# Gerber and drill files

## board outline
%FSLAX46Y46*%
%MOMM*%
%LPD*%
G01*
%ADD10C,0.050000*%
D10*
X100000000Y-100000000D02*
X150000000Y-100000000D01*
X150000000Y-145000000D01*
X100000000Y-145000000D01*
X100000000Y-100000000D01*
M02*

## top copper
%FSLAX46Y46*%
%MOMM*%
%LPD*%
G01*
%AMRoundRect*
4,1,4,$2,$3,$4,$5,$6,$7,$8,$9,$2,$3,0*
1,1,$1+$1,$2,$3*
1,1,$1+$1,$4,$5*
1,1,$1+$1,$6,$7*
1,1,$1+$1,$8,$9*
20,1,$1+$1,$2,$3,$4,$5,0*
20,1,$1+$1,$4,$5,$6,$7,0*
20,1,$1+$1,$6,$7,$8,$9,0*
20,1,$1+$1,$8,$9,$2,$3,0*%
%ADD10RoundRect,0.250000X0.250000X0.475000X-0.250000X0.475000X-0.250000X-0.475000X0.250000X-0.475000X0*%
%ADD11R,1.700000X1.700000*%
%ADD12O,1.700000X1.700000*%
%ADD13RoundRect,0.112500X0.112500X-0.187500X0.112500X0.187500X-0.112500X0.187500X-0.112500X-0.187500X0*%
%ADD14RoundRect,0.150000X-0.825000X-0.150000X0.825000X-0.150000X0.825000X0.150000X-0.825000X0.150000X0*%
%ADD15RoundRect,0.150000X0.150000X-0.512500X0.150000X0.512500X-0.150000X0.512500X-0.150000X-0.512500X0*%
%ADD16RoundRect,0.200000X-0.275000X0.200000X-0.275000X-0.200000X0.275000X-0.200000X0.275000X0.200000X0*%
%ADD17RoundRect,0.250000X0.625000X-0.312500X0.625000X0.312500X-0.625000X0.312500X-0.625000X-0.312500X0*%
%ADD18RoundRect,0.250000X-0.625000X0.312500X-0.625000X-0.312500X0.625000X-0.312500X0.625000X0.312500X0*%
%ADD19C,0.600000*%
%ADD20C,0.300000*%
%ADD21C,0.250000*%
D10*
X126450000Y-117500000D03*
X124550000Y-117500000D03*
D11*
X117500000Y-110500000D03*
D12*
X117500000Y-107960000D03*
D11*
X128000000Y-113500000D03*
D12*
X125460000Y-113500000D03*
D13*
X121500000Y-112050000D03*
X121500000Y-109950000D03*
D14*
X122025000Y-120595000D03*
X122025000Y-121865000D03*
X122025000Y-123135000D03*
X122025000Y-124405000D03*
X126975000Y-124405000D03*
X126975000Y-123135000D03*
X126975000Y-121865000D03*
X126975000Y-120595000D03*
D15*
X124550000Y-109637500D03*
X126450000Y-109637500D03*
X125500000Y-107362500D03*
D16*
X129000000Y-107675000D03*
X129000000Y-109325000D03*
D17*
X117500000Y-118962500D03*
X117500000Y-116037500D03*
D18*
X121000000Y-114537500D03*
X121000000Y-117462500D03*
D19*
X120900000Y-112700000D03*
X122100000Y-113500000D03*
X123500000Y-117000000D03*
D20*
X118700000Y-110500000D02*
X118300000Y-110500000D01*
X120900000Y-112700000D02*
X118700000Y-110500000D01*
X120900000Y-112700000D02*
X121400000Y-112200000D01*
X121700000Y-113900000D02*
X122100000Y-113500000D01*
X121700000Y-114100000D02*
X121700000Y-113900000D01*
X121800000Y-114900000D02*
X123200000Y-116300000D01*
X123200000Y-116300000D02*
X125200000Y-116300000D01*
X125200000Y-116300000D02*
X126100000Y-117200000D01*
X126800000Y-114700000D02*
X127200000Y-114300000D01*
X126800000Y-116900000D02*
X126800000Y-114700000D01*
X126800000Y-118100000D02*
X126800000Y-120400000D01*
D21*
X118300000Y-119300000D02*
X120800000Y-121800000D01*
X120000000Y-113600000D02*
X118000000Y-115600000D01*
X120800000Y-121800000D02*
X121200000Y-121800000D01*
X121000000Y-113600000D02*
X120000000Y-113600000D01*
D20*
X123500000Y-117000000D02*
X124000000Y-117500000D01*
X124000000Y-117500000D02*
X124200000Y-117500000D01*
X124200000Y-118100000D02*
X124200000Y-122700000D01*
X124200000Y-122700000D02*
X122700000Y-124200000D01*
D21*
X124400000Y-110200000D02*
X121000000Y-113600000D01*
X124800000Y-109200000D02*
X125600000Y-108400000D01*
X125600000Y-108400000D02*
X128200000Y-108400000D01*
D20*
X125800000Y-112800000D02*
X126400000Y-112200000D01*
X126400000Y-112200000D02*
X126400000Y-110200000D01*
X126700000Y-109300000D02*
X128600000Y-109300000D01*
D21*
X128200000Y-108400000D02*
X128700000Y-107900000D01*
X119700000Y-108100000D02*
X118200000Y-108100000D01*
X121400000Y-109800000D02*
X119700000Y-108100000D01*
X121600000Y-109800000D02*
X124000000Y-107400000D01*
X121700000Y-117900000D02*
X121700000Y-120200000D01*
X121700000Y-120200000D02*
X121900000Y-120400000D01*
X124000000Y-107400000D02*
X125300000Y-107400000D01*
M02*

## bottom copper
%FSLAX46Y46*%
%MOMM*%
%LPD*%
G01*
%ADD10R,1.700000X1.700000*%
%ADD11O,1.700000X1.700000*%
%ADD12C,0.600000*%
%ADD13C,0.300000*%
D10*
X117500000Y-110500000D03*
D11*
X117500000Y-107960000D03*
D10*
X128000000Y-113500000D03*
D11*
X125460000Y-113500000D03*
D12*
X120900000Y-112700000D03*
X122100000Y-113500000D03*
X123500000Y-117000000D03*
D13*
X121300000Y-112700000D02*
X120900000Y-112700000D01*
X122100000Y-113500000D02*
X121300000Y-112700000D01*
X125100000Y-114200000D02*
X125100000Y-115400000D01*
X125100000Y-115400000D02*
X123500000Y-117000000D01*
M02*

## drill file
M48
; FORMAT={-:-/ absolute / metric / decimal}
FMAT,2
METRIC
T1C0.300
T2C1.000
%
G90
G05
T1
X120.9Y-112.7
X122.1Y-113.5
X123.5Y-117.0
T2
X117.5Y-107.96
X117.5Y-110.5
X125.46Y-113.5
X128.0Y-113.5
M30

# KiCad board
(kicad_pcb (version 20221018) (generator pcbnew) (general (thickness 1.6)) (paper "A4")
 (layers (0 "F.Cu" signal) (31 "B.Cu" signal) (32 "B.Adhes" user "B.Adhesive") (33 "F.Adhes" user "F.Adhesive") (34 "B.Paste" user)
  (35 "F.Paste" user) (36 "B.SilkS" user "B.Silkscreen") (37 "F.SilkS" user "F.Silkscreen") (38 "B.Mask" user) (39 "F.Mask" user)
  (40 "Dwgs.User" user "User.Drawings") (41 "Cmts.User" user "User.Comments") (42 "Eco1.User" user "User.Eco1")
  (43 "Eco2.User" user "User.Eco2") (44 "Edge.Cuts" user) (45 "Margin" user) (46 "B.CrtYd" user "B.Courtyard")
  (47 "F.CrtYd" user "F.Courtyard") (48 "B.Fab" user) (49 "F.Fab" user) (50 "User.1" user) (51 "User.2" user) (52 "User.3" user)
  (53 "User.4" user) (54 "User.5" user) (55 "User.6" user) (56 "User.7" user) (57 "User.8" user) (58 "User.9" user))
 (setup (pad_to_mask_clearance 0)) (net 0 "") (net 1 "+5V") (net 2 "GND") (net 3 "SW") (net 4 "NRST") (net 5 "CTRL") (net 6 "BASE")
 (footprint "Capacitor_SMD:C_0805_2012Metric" (layer "F.Cu") (at 125.5 117.5 180)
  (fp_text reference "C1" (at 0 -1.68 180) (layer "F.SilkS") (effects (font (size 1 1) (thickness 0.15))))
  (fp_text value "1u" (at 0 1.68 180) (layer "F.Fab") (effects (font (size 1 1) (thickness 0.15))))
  (pad "1" smd roundrect (at -0.95 0 180) (size 1 1.45) (layers "F.Cu" "F.Paste" "F.Mask") (roundrect_rratio 0.25) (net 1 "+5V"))
  (pad "2" smd roundrect (at 0.95 0 180) (size 1 1.45) (layers "F.Cu" "F.Paste" "F.Mask") (roundrect_rratio 0.25) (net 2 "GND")))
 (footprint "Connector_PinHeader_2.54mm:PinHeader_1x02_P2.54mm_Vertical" (layer "F.Cu") (at 117.5 110.5 180)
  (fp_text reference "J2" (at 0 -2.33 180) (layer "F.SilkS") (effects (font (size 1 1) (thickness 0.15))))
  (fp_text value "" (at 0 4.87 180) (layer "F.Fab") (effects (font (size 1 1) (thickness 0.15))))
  (pad "1" thru_hole rect (at 0 0 180) (size 1.7 1.7) (drill 1) (layers "*.Cu" "*.Mask") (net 1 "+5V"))
  (pad "2" thru_hole oval (at 0 2.54 180) (size 1.7 1.7) (drill 1) (layers "*.Cu" "*.Mask") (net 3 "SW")))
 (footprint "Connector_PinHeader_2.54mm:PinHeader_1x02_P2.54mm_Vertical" (layer "F.Cu") (at 128 113.5 -90)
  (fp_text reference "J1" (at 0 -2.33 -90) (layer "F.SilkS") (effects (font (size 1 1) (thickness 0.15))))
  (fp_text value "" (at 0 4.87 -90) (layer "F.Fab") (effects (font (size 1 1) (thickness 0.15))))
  (pad "1" thru_hole rect (at 0 0 270) (size 1.7 1.7) (drill 1) (layers "*.Cu" "*.Mask") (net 1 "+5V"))
  (pad "2" thru_hole oval (at 0 2.54 270) (size 1.7 1.7) (drill 1) (layers "*.Cu" "*.Mask") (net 2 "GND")))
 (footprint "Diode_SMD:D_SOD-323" (layer "F.Cu") (at 121.5 111 90)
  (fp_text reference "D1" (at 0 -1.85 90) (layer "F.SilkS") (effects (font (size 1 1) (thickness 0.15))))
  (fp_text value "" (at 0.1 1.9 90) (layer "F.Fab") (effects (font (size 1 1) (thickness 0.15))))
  (pad "1" smd roundrect (at -1.05 0 90) (size 0.6 0.45) (layers "F.Cu" "F.Paste" "F.Mask") (roundrect_rratio 0.25) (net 1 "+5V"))
  (pad "2" smd roundrect (at 1.05 0 90) (size 0.6 0.45) (layers "F.Cu" "F.Paste" "F.Mask") (roundrect_rratio 0.25) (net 3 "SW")))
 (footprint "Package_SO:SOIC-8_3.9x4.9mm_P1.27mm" (layer "F.Cu") (at 124.5 122.5)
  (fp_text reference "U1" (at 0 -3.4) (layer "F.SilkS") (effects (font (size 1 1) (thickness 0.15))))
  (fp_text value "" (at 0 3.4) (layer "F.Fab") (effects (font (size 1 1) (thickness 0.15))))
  (pad "1" smd roundrect (at -2.475 -1.905) (size 1.95 0.6) (layers "F.Cu" "F.Paste" "F.Mask") (roundrect_rratio 0.25) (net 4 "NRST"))
  (pad "2" smd roundrect (at -2.475 -0.635) (size 1.95 0.6) (layers "F.Cu" "F.Paste" "F.Mask") (roundrect_rratio 0.25) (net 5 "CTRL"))
  (pad "3" smd roundrect (at -2.475 0.635) (size 1.95 0.6) (layers "F.Cu" "F.Paste" "F.Mask") (roundrect_rratio 0.25))
  (pad "4" smd roundrect (at -2.475 1.905) (size 1.95 0.6) (layers "F.Cu" "F.Paste" "F.Mask") (roundrect_rratio 0.25) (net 2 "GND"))
  (pad "5" smd roundrect (at 2.475 1.905) (size 1.95 0.6) (layers "F.Cu" "F.Paste" "F.Mask") (roundrect_rratio 0.25))
  (pad "6" smd roundrect (at 2.475 0.635) (size 1.95 0.6) (layers "F.Cu" "F.Paste" "F.Mask") (roundrect_rratio 0.25))
  (pad "7" smd roundrect (at 2.475 -0.635) (size 1.95 0.6) (layers "F.Cu" "F.Paste" "F.Mask") (roundrect_rratio 0.25))
  (pad "8" smd roundrect (at 2.475 -1.905) (size 1.95 0.6) (layers "F.Cu" "F.Paste" "F.Mask") (roundrect_rratio 0.25) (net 1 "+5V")))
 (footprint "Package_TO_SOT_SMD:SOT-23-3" (layer "F.Cu") (at 125.5 108.5 90)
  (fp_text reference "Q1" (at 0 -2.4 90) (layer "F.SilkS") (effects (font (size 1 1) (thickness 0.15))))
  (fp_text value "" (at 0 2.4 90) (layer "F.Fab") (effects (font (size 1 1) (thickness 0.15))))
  (pad "1" smd roundrect (at -1.1375 -0.95 90) (size 1.325 0.6) (layers "F.Cu" "F.Paste" "F.Mask") (roundrect_rratio 0.25) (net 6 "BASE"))
  (pad "2" smd roundrect (at -1.1375 0.95 90) (size 1.325 0.6) (layers "F.Cu" "F.Paste" "F.Mask") (roundrect_rratio 0.25) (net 2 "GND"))
  (pad "3" smd roundrect (at 1.1375 0 90) (size 1.325 0.6) (layers "F.Cu" "F.Paste" "F.Mask") (roundrect_rratio 0.25) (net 3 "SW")))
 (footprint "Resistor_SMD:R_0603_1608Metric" (layer "F.Cu") (at 129 108.5 -90)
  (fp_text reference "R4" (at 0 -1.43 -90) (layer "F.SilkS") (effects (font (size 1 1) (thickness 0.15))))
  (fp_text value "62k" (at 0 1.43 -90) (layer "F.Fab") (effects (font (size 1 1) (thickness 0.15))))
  (pad "1" smd roundrect (at -0.825 0 270) (size 0.8 0.95) (layers "F.Cu" "F.Paste" "F.Mask") (roundrect_rratio 0.25) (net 6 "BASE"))
  (pad "2" smd roundrect (at 0.825 0 270) (size 0.8 0.95) (layers "F.Cu" "F.Paste" "F.Mask") (roundrect_rratio 0.25) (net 2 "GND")))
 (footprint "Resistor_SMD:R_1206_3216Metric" (layer "F.Cu") (at 117.5 117.5 90)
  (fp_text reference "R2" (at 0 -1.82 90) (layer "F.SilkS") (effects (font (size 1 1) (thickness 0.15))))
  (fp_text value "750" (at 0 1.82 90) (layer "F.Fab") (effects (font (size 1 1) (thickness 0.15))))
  (pad "1" smd roundrect (at -1.4625 0 90) (size 1.125 1.75) (layers "F.Cu" "F.Paste" "F.Mask") (roundrect_rratio 0.222222) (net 5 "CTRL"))
  (pad "2" smd roundrect (at 1.4625 0 90) (size 1.125 1.75) (layers "F.Cu" "F.Paste" "F.Mask") (roundrect_rratio 0.222222) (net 6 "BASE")))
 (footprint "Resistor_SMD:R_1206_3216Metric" (layer "F.Cu") (at 121 116 -90)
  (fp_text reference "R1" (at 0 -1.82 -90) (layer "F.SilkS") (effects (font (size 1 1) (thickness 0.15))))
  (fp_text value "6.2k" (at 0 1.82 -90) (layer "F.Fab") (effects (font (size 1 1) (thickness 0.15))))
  (pad "1" smd roundrect (at -1.4625 0 270) (size 1.125 1.75) (layers "F.Cu" "F.Paste" "F.Mask") (roundrect_rratio 0.222222) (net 1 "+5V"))
  (pad "2" smd roundrect (at 1.4625 0 270) (size 1.125 1.75) (layers "F.Cu" "F.Paste" "F.Mask") (roundrect_rratio 0.222222) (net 4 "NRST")))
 (gr_rect (start 100 100) (end 150 145) (stroke (width 0.05) (type default)) (fill none) (layer "Edge.Cuts"))
 (segment (start 118.7 110.5) (end 118.3 110.5) (width 0.3) (layer "F.Cu") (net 1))
 (segment (start 120.9 112.7) (end 118.7 110.5) (width 0.3) (layer "F.Cu") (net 1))
 (segment (start 120.9 112.7) (end 121.4 112.2) (width 0.3) (layer "F.Cu") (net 1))
 (segment (start 121.7 113.9) (end 122.1 113.5) (width 0.3) (layer "F.Cu") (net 1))
 (segment (start 121.7 114.1) (end 121.7 113.9) (width 0.3) (layer "F.Cu") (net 1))
 (segment (start 121.8 114.9) (end 123.2 116.3) (width 0.3) (layer "F.Cu") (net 1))
 (segment (start 123.2 116.3) (end 125.2 116.3) (width 0.3) (layer "F.Cu") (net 1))
 (segment (start 125.2 116.3) (end 126.1 117.2) (width 0.3) (layer "F.Cu") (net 1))
 (segment (start 126.8 114.7) (end 127.2 114.3) (width 0.3) (layer "F.Cu") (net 1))
 (segment (start 126.8 116.9) (end 126.8 114.7) (width 0.3) (layer "F.Cu") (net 1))
 (segment (start 126.8 118.1) (end 126.8 120.4) (width 0.3) (layer "F.Cu") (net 1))
 (via (at 120.9 112.7) (size 0.6) (drill 0.3) (layers "F.Cu" "B.Cu") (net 1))
 (via (at 122.1 113.5) (size 0.6) (drill 0.3) (layers "F.Cu" "B.Cu") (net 1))
 (segment (start 118.3 119.3) (end 120.8 121.8) (width 0.25) (layer "F.Cu") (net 5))
 (segment (start 120 113.6) (end 118 115.6) (width 0.25) (layer "F.Cu") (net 6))
 (segment (start 120.8 121.8) (end 121.2 121.8) (width 0.25) (layer "F.Cu") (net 5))
 (segment (start 121 113.6) (end 120 113.6) (width 0.25) (layer "F.Cu") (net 6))
 (segment (start 121.3 112.7) (end 120.9 112.7) (width 0.3) (layer "B.Cu") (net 1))
 (segment (start 122.1 113.5) (end 121.3 112.7) (width 0.3) (layer "B.Cu") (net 1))
 (segment (start 123.5 117) (end 124 117.5) (width 0.3) (layer "F.Cu") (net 2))
 (segment (start 124 117.5) (end 124.2 117.5) (width 0.3) (layer "F.Cu") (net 2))
 (segment (start 124.2 118.1) (end 124.2 122.7) (width 0.3) (layer "F.Cu") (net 2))
 (segment (start 124.2 122.7) (end 122.7 124.2) (width 0.3) (layer "F.Cu") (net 2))
 (segment (start 124.4 110.2) (end 121 113.6) (width 0.25) (layer "F.Cu") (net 6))
 (segment (start 124.8 109.2) (end 125.6 108.4) (width 0.25) (layer "F.Cu") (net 6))
 (segment (start 125.6 108.4) (end 128.2 108.4) (width 0.25) (layer "F.Cu") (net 6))
 (segment (start 125.8 112.8) (end 126.4 112.2) (width 0.3) (layer "F.Cu") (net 2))
 (segment (start 126.4 112.2) (end 126.4 110.2) (width 0.3) (layer "F.Cu") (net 2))
 (segment (start 126.7 109.3) (end 128.6 109.3) (width 0.3) (layer "F.Cu") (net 2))
 (segment (start 128.2 108.4) (end 128.7 107.9) (width 0.25) (layer "F.Cu") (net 6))
 (via (at 123.5 117) (size 0.6) (drill 0.3) (layers "F.Cu" "B.Cu") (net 2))
 (segment (start 119.7 108.1) (end 118.2 108.1) (width 0.25) (layer "F.Cu") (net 3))
 (segment (start 121.4 109.8) (end 119.7 108.1) (width 0.25) (layer "F.Cu") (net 3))
 (segment (start 121.6 109.8) (end 124 107.4) (width 0.25) (layer "F.Cu") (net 3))
 (segment (start 121.7 117.9) (end 121.7 120.2) (width 0.25) (layer "F.Cu") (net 4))
 (segment (start 121.7 120.2) (end 121.9 120.4) (width 0.25) (layer "F.Cu") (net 4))
 (segment (start 124 107.4) (end 125.3 107.4) (width 0.25) (layer "F.Cu") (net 3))
 (segment (start 125.1 114.2) (end 125.1 115.4) (width 0.3) (layer "B.Cu") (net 2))
 (segment (start 125.1 115.4) (end 123.5 117) (width 0.3) (layer "B.Cu") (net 2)))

